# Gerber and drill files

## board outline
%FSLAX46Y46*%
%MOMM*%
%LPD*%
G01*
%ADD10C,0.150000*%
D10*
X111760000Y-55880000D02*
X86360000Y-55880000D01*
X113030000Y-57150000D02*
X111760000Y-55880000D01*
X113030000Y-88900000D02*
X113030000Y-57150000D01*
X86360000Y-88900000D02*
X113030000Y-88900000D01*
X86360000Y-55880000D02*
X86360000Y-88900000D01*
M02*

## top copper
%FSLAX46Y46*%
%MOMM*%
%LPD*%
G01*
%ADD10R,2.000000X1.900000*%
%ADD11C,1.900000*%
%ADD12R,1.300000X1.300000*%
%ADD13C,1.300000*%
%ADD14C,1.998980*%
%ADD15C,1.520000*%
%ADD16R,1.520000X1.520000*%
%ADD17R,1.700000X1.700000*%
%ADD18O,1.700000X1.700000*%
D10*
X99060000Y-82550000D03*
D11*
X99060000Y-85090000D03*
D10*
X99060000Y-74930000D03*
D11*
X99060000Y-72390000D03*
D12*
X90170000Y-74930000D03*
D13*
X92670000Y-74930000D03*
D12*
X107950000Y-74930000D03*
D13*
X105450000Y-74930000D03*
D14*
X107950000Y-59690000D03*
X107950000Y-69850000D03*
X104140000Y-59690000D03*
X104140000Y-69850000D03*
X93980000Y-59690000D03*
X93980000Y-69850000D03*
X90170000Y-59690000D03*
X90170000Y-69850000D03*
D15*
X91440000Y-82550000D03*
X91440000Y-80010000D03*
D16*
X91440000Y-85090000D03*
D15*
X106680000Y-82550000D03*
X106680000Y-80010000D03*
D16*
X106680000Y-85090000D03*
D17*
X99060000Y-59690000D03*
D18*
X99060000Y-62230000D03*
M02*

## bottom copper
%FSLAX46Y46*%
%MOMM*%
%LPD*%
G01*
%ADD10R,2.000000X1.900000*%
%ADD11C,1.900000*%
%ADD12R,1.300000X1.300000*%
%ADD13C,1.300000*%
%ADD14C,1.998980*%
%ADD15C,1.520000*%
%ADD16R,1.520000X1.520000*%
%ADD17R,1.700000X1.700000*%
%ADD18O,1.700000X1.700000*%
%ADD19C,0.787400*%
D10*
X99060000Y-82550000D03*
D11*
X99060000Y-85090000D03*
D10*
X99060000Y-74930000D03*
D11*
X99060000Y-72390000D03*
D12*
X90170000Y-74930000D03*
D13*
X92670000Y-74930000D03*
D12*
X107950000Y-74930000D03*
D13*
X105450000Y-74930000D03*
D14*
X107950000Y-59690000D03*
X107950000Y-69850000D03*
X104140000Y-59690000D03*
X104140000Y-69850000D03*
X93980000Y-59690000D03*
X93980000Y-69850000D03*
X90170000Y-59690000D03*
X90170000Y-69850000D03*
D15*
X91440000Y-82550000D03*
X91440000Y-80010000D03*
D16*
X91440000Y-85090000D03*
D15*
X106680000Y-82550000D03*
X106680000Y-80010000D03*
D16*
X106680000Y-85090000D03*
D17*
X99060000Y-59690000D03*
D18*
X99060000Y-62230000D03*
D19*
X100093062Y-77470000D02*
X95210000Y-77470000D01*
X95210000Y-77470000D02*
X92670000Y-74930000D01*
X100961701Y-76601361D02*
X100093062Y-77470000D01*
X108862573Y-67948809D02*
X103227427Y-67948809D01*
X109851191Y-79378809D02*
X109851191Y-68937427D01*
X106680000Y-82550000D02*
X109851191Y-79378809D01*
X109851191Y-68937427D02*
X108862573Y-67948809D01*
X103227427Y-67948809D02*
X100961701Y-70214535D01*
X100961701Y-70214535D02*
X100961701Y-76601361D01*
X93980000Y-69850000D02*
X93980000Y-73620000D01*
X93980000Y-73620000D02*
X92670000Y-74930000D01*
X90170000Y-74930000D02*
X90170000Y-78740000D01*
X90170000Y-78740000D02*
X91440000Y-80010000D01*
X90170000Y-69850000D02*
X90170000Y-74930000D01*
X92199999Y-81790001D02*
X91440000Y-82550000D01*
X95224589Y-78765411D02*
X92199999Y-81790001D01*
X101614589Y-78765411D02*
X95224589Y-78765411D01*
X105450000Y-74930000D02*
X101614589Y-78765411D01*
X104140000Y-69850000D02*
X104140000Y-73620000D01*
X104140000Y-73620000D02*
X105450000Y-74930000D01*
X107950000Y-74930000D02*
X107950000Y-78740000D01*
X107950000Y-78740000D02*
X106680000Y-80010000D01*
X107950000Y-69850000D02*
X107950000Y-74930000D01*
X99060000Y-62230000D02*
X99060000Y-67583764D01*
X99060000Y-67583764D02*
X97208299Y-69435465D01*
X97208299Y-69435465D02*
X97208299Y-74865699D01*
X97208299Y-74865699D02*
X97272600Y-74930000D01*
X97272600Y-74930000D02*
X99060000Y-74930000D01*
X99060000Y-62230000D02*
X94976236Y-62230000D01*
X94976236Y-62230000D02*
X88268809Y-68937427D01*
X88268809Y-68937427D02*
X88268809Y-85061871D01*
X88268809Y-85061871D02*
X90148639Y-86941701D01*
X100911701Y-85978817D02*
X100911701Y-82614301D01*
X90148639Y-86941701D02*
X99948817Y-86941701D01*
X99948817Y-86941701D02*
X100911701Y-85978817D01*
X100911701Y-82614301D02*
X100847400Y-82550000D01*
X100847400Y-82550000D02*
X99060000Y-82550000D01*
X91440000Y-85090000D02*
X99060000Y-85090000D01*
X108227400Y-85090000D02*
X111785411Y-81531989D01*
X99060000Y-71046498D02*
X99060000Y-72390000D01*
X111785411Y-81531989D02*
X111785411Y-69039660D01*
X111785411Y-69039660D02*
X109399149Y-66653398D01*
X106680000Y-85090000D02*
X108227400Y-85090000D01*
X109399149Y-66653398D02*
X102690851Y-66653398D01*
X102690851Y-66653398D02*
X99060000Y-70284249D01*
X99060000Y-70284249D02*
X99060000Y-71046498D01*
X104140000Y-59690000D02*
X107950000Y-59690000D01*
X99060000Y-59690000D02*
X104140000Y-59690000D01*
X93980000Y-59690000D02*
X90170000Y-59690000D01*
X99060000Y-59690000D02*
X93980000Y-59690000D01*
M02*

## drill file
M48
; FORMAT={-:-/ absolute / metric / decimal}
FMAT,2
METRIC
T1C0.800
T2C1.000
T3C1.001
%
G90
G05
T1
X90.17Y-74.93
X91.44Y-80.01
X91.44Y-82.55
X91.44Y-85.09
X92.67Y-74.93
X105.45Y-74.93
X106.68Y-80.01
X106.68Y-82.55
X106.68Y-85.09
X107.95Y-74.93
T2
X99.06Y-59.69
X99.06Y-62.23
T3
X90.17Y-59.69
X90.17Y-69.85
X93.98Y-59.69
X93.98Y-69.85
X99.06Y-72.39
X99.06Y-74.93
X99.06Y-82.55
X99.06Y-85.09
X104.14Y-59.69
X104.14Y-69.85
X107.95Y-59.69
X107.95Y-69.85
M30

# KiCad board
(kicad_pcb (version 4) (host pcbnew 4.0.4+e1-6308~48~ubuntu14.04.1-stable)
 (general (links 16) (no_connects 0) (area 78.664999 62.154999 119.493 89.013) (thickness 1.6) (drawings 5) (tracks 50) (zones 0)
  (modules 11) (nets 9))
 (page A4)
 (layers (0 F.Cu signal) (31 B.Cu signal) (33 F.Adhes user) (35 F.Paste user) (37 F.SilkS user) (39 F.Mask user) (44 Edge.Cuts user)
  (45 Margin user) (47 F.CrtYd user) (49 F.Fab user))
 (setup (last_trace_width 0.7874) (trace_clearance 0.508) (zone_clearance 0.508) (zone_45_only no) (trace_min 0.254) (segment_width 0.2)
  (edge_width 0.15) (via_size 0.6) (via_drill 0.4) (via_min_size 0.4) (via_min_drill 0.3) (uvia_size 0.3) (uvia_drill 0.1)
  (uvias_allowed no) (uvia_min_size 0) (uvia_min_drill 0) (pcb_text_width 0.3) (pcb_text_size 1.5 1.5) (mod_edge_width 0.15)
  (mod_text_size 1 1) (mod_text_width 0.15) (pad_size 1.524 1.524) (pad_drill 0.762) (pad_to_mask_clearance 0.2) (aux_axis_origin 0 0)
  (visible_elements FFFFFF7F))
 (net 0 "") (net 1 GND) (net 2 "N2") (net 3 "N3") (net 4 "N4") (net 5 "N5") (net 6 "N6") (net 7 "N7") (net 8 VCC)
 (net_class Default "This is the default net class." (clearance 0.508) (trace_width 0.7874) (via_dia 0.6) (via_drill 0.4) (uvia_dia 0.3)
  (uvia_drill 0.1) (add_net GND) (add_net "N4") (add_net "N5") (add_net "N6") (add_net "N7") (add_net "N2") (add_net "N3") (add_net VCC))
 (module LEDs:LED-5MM (layer F.Cu) (at 99.06 82.55 270)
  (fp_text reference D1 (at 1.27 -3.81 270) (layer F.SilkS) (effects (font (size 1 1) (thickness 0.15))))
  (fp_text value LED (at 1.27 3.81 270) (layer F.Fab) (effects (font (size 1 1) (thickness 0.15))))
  (pad 1 thru_hole rect (at 0 0) (size 2 1.9) (drill 1.00076) (layers *.Cu *.Mask F.SilkS) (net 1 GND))
  (pad 2 thru_hole circle (at 2.54 0 270) (size 1.9 1.9) (drill 1.00076) (layers *.Cu *.Mask F.SilkS) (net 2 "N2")))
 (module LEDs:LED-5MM (layer F.Cu) (at 99.06 74.93 90)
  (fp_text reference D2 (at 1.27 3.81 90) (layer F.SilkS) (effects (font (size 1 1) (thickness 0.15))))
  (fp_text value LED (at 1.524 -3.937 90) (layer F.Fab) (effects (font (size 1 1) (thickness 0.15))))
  (pad 1 thru_hole rect (at 0 0 180) (size 2 1.9) (drill 1.00076) (layers *.Cu *.Mask F.SilkS) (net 1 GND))
  (pad 2 thru_hole circle (at 2.54 0 90) (size 1.9 1.9) (drill 1.00076) (layers *.Cu *.Mask F.SilkS) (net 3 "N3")))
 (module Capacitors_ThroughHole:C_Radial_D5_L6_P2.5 (layer F.Cu) (at 90.17 74.93)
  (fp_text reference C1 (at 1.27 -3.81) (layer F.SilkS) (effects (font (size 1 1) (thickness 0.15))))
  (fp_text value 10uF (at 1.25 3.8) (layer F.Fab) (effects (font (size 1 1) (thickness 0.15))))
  (pad 1 thru_hole rect (at 0 0) (size 1.3 1.3) (drill 0.8) (layers *.Cu *.Mask F.SilkS) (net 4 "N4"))
  (pad 2 thru_hole circle (at 2.5 0) (size 1.3 1.3) (drill 0.8) (layers *.Cu *.Mask F.SilkS) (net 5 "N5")))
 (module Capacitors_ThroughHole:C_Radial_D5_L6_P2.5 (layer F.Cu) (at 107.95 74.93 180)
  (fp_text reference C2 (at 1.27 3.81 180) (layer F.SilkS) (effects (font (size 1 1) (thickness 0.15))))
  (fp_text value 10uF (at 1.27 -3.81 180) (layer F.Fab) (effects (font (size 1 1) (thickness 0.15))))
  (pad 1 thru_hole rect (at 0 0 180) (size 1.3 1.3) (drill 0.8) (layers *.Cu *.Mask F.SilkS) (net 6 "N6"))
  (pad 2 thru_hole circle (at 2.5 0 180) (size 1.3 1.3) (drill 0.8) (layers *.Cu *.Mask F.SilkS) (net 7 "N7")))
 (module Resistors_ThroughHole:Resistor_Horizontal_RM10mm (layer F.Cu) (at 107.95 59.69 270)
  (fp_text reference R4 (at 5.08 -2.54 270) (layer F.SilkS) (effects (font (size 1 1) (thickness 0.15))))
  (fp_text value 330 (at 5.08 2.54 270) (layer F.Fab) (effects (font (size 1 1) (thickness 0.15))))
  (pad 1 thru_hole circle (at 0 0 270) (size 1.99898 1.99898) (drill 1.00076) (layers *.Cu *.SilkS *.Mask) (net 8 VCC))
  (pad 2 thru_hole circle (at 10.16 0 270) (size 1.99898 1.99898) (drill 1.00076) (layers *.Cu *.SilkS *.Mask) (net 6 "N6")))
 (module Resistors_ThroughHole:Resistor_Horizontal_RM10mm (layer F.Cu) (at 104.14 59.69 270)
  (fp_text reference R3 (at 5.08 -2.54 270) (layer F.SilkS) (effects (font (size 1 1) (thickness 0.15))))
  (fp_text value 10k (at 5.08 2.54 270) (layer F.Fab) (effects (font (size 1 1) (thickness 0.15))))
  (pad 1 thru_hole circle (at 0 0 270) (size 1.99898 1.99898) (drill 1.00076) (layers *.Cu *.SilkS *.Mask) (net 8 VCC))
  (pad 2 thru_hole circle (at 10.16 0 270) (size 1.99898 1.99898) (drill 1.00076) (layers *.Cu *.SilkS *.Mask) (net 7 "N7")))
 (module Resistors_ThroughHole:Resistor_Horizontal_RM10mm (layer F.Cu) (at 93.98 59.69 270)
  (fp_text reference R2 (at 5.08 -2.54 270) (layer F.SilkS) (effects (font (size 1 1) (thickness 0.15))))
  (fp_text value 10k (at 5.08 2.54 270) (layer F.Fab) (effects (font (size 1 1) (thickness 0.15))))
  (pad 1 thru_hole circle (at 0 0 270) (size 1.99898 1.99898) (drill 1.00076) (layers *.Cu *.SilkS *.Mask) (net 8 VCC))
  (pad 2 thru_hole circle (at 10.16 0 270) (size 1.99898 1.99898) (drill 1.00076) (layers *.Cu *.SilkS *.Mask) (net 5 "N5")))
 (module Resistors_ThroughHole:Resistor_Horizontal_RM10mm (layer F.Cu) (at 90.17 59.69 270)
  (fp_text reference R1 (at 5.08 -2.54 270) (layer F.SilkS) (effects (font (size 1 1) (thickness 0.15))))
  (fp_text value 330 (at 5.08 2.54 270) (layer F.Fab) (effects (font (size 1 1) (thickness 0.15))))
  (pad 1 thru_hole circle (at 0 0 270) (size 1.99898 1.99898) (drill 1.00076) (layers *.Cu *.SilkS *.Mask) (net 8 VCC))
  (pad 2 thru_hole circle (at 10.16 0 270) (size 1.99898 1.99898) (drill 1.00076) (layers *.Cu *.SilkS *.Mask) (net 4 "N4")))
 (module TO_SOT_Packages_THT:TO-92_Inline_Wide (layer F.Cu) (at 91.44 85.09 90)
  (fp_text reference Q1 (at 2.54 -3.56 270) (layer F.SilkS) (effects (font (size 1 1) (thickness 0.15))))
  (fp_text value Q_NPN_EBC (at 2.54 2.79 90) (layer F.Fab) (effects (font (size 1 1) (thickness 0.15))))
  (pad 2 thru_hole circle (at 2.54 0 180) (size 1.52 1.52) (drill 0.8) (layers *.Cu *.Mask) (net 7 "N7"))
  (pad 3 thru_hole circle (at 5.08 0 180) (size 1.52 1.52) (drill 0.8) (layers *.Cu *.Mask) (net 4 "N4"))
  (pad 1 thru_hole rect (at 0 0 180) (size 1.52 1.52) (drill 0.8) (layers *.Cu *.Mask) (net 2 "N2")))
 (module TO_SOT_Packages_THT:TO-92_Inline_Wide (layer F.Cu) (at 106.68 85.09 90)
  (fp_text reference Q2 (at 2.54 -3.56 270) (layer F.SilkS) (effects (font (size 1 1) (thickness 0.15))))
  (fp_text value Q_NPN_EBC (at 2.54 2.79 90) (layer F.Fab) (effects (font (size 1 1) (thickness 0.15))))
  (pad 2 thru_hole circle (at 2.54 0 180) (size 1.52 1.52) (drill 0.8) (layers *.Cu *.Mask) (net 5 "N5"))
  (pad 3 thru_hole circle (at 5.08 0 180) (size 1.52 1.52) (drill 0.8) (layers *.Cu *.Mask) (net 6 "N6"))
  (pad 1 thru_hole rect (at 0 0 180) (size 1.52 1.52) (drill 0.8) (layers *.Cu *.Mask) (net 3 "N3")))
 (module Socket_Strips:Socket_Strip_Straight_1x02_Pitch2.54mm (layer F.Cu) (at 99.06 59.69)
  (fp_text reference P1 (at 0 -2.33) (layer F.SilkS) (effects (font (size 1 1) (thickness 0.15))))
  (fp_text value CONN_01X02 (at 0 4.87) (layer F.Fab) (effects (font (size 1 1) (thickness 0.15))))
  (pad 1 thru_hole rect (at 0 0) (size 1.7 1.7) (drill 1) (layers *.Cu *.Mask) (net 8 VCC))
  (pad 2 thru_hole oval (at 0 2.54) (size 1.7 1.7) (drill 1) (layers *.Cu *.Mask) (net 1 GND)))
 (gr_line (start 111.76 55.88) (end 86.36 55.88) (angle 90) (layer Edge.Cuts) (width 0.15))
 (gr_line (start 113.03 57.15) (end 111.76 55.88) (angle 90) (layer Edge.Cuts) (width 0.15))
 (gr_line (start 113.03 88.9) (end 113.03 57.15) (angle 90) (layer Edge.Cuts) (width 0.15))
 (gr_line (start 86.36 88.9) (end 113.03 88.9) (angle 90) (layer Edge.Cuts) (width 0.15))
 (gr_line (start 86.36 55.88) (end 86.36 88.9) (angle 90) (layer Edge.Cuts) (width 0.15))
 (segment (start 100.093062 77.47) (end 95.21 77.47) (width 0.7874) (layer B.Cu) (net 5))
 (segment (start 95.21 77.47) (end 92.67 74.93) (width 0.7874) (layer B.Cu) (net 5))
 (segment (start 100.961701 76.601361) (end 100.093062 77.47) (width 0.7874) (layer B.Cu) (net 5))
 (segment (start 108.862573 67.948809) (end 103.227427 67.948809) (width 0.7874) (layer B.Cu) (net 5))
 (segment (start 109.851191 79.378809) (end 109.851191 68.937427) (width 0.7874) (layer B.Cu) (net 5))
 (segment (start 106.68 82.55) (end 109.851191 79.378809) (width 0.7874) (layer B.Cu) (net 5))
 (segment (start 109.851191 68.937427) (end 108.862573 67.948809) (width 0.7874) (layer B.Cu) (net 5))
 (segment (start 103.227427 67.948809) (end 100.961701 70.214535) (width 0.7874) (layer B.Cu) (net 5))
 (segment (start 100.961701 70.214535) (end 100.961701 76.601361) (width 0.7874) (layer B.Cu) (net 5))
 (segment (start 93.98 69.85) (end 93.98 73.62) (width 0.7874) (layer B.Cu) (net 5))
 (segment (start 93.98 73.62) (end 92.67 74.93) (width 0.7874) (layer B.Cu) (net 5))
 (segment (start 90.17 74.93) (end 90.17 78.74) (width 0.7874) (layer B.Cu) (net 4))
 (segment (start 90.17 78.74) (end 91.44 80.01) (width 0.7874) (layer B.Cu) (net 4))
 (segment (start 90.17 69.85) (end 90.17 74.93) (width 0.7874) (layer B.Cu) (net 4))
 (segment (start 92.199999 81.790001) (end 91.44 82.55) (width 0.7874) (layer B.Cu) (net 7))
 (segment (start 95.224589 78.765411) (end 92.199999 81.790001) (width 0.7874) (layer B.Cu) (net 7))
 (segment (start 101.614589 78.765411) (end 95.224589 78.765411) (width 0.7874) (layer B.Cu) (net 7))
 (segment (start 105.45 74.93) (end 101.614589 78.765411) (width 0.7874) (layer B.Cu) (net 7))
 (segment (start 104.14 69.85) (end 104.14 73.62) (width 0.7874) (layer B.Cu) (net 7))
 (segment (start 104.14 73.62) (end 105.45 74.93) (width 0.7874) (layer B.Cu) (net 7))
 (segment (start 107.95 74.93) (end 107.95 78.74) (width 0.7874) (layer B.Cu) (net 6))
 (segment (start 107.95 78.74) (end 106.68 80.01) (width 0.7874) (layer B.Cu) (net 6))
 (segment (start 107.95 69.85) (end 107.95 74.93) (width 0.7874) (layer B.Cu) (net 6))
 (segment (start 99.06 62.23) (end 99.06 67.583764) (width 0.7874) (layer B.Cu) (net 1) (status 10))
 (segment (start 99.06 67.583764) (end 97.208299 69.435465) (width 0.7874) (layer B.Cu) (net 1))
 (segment (start 97.208299 69.435465) (end 97.208299 74.865699) (width 0.7874) (layer B.Cu) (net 1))
 (segment (start 97.208299 74.865699) (end 97.2726 74.93) (width 0.7874) (layer B.Cu) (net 1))
 (segment (start 97.2726 74.93) (end 99.06 74.93) (width 0.7874) (layer B.Cu) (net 1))
 (segment (start 99.06 62.23) (end 94.976236 62.23) (width 0.7874) (layer B.Cu) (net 1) (status 10))
 (segment (start 94.976236 62.23) (end 88.268809 68.937427) (width 0.7874) (layer B.Cu) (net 1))
 (segment (start 88.268809 68.937427) (end 88.268809 85.061871) (width 0.7874) (layer B.Cu) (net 1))
 (segment (start 88.268809 85.061871) (end 90.148639 86.941701) (width 0.7874) (layer B.Cu) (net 1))
 (segment (start 100.911701 85.978817) (end 100.911701 82.614301) (width 0.7874) (layer B.Cu) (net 1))
 (segment (start 90.148639 86.941701) (end 99.948817 86.941701) (width 0.7874) (layer B.Cu) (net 1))
 (segment (start 99.948817 86.941701) (end 100.911701 85.978817) (width 0.7874) (layer B.Cu) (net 1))
 (segment (start 100.911701 82.614301) (end 100.8474 82.55) (width 0.7874) (layer B.Cu) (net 1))
 (segment (start 100.8474 82.55) (end 99.06 82.55) (width 0.7874) (layer B.Cu) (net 1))
 (segment (start 91.44 85.09) (end 99.06 85.09) (width 0.7874) (layer B.Cu) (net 2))
 (segment (start 108.2274 85.09) (end 111.785411 81.531989) (width 0.7874) (layer B.Cu) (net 3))
 (segment (start 99.06 71.046498) (end 99.06 72.39) (width 0.7874) (layer B.Cu) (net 3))
 (segment (start 111.785411 81.531989) (end 111.785411 69.03966) (width 0.7874) (layer B.Cu) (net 3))
 (segment (start 111.785411 69.03966) (end 109.399149 66.653398) (width 0.7874) (layer B.Cu) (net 3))
 (segment (start 106.68 85.09) (end 108.2274 85.09) (width 0.7874) (layer B.Cu) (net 3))
 (segment (start 109.399149 66.653398) (end 102.690851 66.653398) (width 0.7874) (layer B.Cu) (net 3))
 (segment (start 102.690851 66.653398) (end 99.06 70.284249) (width 0.7874) (layer B.Cu) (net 3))
 (segment (start 99.06 70.284249) (end 99.06 71.046498) (width 0.7874) (layer B.Cu) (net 3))
 (segment (start 104.14 59.69) (end 107.95 59.69) (width 0.7874) (layer B.Cu) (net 8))
 (segment (start 99.06 59.69) (end 104.14 59.69) (width 0.7874) (layer B.Cu) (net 8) (status 10))
 (segment (start 93.98 59.69) (end 90.17 59.69) (width 0.7874) (layer B.Cu) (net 8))
 (segment (start 99.06 59.69) (end 93.98 59.69) (width 0.7874) (layer B.Cu) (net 8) (status 10)))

